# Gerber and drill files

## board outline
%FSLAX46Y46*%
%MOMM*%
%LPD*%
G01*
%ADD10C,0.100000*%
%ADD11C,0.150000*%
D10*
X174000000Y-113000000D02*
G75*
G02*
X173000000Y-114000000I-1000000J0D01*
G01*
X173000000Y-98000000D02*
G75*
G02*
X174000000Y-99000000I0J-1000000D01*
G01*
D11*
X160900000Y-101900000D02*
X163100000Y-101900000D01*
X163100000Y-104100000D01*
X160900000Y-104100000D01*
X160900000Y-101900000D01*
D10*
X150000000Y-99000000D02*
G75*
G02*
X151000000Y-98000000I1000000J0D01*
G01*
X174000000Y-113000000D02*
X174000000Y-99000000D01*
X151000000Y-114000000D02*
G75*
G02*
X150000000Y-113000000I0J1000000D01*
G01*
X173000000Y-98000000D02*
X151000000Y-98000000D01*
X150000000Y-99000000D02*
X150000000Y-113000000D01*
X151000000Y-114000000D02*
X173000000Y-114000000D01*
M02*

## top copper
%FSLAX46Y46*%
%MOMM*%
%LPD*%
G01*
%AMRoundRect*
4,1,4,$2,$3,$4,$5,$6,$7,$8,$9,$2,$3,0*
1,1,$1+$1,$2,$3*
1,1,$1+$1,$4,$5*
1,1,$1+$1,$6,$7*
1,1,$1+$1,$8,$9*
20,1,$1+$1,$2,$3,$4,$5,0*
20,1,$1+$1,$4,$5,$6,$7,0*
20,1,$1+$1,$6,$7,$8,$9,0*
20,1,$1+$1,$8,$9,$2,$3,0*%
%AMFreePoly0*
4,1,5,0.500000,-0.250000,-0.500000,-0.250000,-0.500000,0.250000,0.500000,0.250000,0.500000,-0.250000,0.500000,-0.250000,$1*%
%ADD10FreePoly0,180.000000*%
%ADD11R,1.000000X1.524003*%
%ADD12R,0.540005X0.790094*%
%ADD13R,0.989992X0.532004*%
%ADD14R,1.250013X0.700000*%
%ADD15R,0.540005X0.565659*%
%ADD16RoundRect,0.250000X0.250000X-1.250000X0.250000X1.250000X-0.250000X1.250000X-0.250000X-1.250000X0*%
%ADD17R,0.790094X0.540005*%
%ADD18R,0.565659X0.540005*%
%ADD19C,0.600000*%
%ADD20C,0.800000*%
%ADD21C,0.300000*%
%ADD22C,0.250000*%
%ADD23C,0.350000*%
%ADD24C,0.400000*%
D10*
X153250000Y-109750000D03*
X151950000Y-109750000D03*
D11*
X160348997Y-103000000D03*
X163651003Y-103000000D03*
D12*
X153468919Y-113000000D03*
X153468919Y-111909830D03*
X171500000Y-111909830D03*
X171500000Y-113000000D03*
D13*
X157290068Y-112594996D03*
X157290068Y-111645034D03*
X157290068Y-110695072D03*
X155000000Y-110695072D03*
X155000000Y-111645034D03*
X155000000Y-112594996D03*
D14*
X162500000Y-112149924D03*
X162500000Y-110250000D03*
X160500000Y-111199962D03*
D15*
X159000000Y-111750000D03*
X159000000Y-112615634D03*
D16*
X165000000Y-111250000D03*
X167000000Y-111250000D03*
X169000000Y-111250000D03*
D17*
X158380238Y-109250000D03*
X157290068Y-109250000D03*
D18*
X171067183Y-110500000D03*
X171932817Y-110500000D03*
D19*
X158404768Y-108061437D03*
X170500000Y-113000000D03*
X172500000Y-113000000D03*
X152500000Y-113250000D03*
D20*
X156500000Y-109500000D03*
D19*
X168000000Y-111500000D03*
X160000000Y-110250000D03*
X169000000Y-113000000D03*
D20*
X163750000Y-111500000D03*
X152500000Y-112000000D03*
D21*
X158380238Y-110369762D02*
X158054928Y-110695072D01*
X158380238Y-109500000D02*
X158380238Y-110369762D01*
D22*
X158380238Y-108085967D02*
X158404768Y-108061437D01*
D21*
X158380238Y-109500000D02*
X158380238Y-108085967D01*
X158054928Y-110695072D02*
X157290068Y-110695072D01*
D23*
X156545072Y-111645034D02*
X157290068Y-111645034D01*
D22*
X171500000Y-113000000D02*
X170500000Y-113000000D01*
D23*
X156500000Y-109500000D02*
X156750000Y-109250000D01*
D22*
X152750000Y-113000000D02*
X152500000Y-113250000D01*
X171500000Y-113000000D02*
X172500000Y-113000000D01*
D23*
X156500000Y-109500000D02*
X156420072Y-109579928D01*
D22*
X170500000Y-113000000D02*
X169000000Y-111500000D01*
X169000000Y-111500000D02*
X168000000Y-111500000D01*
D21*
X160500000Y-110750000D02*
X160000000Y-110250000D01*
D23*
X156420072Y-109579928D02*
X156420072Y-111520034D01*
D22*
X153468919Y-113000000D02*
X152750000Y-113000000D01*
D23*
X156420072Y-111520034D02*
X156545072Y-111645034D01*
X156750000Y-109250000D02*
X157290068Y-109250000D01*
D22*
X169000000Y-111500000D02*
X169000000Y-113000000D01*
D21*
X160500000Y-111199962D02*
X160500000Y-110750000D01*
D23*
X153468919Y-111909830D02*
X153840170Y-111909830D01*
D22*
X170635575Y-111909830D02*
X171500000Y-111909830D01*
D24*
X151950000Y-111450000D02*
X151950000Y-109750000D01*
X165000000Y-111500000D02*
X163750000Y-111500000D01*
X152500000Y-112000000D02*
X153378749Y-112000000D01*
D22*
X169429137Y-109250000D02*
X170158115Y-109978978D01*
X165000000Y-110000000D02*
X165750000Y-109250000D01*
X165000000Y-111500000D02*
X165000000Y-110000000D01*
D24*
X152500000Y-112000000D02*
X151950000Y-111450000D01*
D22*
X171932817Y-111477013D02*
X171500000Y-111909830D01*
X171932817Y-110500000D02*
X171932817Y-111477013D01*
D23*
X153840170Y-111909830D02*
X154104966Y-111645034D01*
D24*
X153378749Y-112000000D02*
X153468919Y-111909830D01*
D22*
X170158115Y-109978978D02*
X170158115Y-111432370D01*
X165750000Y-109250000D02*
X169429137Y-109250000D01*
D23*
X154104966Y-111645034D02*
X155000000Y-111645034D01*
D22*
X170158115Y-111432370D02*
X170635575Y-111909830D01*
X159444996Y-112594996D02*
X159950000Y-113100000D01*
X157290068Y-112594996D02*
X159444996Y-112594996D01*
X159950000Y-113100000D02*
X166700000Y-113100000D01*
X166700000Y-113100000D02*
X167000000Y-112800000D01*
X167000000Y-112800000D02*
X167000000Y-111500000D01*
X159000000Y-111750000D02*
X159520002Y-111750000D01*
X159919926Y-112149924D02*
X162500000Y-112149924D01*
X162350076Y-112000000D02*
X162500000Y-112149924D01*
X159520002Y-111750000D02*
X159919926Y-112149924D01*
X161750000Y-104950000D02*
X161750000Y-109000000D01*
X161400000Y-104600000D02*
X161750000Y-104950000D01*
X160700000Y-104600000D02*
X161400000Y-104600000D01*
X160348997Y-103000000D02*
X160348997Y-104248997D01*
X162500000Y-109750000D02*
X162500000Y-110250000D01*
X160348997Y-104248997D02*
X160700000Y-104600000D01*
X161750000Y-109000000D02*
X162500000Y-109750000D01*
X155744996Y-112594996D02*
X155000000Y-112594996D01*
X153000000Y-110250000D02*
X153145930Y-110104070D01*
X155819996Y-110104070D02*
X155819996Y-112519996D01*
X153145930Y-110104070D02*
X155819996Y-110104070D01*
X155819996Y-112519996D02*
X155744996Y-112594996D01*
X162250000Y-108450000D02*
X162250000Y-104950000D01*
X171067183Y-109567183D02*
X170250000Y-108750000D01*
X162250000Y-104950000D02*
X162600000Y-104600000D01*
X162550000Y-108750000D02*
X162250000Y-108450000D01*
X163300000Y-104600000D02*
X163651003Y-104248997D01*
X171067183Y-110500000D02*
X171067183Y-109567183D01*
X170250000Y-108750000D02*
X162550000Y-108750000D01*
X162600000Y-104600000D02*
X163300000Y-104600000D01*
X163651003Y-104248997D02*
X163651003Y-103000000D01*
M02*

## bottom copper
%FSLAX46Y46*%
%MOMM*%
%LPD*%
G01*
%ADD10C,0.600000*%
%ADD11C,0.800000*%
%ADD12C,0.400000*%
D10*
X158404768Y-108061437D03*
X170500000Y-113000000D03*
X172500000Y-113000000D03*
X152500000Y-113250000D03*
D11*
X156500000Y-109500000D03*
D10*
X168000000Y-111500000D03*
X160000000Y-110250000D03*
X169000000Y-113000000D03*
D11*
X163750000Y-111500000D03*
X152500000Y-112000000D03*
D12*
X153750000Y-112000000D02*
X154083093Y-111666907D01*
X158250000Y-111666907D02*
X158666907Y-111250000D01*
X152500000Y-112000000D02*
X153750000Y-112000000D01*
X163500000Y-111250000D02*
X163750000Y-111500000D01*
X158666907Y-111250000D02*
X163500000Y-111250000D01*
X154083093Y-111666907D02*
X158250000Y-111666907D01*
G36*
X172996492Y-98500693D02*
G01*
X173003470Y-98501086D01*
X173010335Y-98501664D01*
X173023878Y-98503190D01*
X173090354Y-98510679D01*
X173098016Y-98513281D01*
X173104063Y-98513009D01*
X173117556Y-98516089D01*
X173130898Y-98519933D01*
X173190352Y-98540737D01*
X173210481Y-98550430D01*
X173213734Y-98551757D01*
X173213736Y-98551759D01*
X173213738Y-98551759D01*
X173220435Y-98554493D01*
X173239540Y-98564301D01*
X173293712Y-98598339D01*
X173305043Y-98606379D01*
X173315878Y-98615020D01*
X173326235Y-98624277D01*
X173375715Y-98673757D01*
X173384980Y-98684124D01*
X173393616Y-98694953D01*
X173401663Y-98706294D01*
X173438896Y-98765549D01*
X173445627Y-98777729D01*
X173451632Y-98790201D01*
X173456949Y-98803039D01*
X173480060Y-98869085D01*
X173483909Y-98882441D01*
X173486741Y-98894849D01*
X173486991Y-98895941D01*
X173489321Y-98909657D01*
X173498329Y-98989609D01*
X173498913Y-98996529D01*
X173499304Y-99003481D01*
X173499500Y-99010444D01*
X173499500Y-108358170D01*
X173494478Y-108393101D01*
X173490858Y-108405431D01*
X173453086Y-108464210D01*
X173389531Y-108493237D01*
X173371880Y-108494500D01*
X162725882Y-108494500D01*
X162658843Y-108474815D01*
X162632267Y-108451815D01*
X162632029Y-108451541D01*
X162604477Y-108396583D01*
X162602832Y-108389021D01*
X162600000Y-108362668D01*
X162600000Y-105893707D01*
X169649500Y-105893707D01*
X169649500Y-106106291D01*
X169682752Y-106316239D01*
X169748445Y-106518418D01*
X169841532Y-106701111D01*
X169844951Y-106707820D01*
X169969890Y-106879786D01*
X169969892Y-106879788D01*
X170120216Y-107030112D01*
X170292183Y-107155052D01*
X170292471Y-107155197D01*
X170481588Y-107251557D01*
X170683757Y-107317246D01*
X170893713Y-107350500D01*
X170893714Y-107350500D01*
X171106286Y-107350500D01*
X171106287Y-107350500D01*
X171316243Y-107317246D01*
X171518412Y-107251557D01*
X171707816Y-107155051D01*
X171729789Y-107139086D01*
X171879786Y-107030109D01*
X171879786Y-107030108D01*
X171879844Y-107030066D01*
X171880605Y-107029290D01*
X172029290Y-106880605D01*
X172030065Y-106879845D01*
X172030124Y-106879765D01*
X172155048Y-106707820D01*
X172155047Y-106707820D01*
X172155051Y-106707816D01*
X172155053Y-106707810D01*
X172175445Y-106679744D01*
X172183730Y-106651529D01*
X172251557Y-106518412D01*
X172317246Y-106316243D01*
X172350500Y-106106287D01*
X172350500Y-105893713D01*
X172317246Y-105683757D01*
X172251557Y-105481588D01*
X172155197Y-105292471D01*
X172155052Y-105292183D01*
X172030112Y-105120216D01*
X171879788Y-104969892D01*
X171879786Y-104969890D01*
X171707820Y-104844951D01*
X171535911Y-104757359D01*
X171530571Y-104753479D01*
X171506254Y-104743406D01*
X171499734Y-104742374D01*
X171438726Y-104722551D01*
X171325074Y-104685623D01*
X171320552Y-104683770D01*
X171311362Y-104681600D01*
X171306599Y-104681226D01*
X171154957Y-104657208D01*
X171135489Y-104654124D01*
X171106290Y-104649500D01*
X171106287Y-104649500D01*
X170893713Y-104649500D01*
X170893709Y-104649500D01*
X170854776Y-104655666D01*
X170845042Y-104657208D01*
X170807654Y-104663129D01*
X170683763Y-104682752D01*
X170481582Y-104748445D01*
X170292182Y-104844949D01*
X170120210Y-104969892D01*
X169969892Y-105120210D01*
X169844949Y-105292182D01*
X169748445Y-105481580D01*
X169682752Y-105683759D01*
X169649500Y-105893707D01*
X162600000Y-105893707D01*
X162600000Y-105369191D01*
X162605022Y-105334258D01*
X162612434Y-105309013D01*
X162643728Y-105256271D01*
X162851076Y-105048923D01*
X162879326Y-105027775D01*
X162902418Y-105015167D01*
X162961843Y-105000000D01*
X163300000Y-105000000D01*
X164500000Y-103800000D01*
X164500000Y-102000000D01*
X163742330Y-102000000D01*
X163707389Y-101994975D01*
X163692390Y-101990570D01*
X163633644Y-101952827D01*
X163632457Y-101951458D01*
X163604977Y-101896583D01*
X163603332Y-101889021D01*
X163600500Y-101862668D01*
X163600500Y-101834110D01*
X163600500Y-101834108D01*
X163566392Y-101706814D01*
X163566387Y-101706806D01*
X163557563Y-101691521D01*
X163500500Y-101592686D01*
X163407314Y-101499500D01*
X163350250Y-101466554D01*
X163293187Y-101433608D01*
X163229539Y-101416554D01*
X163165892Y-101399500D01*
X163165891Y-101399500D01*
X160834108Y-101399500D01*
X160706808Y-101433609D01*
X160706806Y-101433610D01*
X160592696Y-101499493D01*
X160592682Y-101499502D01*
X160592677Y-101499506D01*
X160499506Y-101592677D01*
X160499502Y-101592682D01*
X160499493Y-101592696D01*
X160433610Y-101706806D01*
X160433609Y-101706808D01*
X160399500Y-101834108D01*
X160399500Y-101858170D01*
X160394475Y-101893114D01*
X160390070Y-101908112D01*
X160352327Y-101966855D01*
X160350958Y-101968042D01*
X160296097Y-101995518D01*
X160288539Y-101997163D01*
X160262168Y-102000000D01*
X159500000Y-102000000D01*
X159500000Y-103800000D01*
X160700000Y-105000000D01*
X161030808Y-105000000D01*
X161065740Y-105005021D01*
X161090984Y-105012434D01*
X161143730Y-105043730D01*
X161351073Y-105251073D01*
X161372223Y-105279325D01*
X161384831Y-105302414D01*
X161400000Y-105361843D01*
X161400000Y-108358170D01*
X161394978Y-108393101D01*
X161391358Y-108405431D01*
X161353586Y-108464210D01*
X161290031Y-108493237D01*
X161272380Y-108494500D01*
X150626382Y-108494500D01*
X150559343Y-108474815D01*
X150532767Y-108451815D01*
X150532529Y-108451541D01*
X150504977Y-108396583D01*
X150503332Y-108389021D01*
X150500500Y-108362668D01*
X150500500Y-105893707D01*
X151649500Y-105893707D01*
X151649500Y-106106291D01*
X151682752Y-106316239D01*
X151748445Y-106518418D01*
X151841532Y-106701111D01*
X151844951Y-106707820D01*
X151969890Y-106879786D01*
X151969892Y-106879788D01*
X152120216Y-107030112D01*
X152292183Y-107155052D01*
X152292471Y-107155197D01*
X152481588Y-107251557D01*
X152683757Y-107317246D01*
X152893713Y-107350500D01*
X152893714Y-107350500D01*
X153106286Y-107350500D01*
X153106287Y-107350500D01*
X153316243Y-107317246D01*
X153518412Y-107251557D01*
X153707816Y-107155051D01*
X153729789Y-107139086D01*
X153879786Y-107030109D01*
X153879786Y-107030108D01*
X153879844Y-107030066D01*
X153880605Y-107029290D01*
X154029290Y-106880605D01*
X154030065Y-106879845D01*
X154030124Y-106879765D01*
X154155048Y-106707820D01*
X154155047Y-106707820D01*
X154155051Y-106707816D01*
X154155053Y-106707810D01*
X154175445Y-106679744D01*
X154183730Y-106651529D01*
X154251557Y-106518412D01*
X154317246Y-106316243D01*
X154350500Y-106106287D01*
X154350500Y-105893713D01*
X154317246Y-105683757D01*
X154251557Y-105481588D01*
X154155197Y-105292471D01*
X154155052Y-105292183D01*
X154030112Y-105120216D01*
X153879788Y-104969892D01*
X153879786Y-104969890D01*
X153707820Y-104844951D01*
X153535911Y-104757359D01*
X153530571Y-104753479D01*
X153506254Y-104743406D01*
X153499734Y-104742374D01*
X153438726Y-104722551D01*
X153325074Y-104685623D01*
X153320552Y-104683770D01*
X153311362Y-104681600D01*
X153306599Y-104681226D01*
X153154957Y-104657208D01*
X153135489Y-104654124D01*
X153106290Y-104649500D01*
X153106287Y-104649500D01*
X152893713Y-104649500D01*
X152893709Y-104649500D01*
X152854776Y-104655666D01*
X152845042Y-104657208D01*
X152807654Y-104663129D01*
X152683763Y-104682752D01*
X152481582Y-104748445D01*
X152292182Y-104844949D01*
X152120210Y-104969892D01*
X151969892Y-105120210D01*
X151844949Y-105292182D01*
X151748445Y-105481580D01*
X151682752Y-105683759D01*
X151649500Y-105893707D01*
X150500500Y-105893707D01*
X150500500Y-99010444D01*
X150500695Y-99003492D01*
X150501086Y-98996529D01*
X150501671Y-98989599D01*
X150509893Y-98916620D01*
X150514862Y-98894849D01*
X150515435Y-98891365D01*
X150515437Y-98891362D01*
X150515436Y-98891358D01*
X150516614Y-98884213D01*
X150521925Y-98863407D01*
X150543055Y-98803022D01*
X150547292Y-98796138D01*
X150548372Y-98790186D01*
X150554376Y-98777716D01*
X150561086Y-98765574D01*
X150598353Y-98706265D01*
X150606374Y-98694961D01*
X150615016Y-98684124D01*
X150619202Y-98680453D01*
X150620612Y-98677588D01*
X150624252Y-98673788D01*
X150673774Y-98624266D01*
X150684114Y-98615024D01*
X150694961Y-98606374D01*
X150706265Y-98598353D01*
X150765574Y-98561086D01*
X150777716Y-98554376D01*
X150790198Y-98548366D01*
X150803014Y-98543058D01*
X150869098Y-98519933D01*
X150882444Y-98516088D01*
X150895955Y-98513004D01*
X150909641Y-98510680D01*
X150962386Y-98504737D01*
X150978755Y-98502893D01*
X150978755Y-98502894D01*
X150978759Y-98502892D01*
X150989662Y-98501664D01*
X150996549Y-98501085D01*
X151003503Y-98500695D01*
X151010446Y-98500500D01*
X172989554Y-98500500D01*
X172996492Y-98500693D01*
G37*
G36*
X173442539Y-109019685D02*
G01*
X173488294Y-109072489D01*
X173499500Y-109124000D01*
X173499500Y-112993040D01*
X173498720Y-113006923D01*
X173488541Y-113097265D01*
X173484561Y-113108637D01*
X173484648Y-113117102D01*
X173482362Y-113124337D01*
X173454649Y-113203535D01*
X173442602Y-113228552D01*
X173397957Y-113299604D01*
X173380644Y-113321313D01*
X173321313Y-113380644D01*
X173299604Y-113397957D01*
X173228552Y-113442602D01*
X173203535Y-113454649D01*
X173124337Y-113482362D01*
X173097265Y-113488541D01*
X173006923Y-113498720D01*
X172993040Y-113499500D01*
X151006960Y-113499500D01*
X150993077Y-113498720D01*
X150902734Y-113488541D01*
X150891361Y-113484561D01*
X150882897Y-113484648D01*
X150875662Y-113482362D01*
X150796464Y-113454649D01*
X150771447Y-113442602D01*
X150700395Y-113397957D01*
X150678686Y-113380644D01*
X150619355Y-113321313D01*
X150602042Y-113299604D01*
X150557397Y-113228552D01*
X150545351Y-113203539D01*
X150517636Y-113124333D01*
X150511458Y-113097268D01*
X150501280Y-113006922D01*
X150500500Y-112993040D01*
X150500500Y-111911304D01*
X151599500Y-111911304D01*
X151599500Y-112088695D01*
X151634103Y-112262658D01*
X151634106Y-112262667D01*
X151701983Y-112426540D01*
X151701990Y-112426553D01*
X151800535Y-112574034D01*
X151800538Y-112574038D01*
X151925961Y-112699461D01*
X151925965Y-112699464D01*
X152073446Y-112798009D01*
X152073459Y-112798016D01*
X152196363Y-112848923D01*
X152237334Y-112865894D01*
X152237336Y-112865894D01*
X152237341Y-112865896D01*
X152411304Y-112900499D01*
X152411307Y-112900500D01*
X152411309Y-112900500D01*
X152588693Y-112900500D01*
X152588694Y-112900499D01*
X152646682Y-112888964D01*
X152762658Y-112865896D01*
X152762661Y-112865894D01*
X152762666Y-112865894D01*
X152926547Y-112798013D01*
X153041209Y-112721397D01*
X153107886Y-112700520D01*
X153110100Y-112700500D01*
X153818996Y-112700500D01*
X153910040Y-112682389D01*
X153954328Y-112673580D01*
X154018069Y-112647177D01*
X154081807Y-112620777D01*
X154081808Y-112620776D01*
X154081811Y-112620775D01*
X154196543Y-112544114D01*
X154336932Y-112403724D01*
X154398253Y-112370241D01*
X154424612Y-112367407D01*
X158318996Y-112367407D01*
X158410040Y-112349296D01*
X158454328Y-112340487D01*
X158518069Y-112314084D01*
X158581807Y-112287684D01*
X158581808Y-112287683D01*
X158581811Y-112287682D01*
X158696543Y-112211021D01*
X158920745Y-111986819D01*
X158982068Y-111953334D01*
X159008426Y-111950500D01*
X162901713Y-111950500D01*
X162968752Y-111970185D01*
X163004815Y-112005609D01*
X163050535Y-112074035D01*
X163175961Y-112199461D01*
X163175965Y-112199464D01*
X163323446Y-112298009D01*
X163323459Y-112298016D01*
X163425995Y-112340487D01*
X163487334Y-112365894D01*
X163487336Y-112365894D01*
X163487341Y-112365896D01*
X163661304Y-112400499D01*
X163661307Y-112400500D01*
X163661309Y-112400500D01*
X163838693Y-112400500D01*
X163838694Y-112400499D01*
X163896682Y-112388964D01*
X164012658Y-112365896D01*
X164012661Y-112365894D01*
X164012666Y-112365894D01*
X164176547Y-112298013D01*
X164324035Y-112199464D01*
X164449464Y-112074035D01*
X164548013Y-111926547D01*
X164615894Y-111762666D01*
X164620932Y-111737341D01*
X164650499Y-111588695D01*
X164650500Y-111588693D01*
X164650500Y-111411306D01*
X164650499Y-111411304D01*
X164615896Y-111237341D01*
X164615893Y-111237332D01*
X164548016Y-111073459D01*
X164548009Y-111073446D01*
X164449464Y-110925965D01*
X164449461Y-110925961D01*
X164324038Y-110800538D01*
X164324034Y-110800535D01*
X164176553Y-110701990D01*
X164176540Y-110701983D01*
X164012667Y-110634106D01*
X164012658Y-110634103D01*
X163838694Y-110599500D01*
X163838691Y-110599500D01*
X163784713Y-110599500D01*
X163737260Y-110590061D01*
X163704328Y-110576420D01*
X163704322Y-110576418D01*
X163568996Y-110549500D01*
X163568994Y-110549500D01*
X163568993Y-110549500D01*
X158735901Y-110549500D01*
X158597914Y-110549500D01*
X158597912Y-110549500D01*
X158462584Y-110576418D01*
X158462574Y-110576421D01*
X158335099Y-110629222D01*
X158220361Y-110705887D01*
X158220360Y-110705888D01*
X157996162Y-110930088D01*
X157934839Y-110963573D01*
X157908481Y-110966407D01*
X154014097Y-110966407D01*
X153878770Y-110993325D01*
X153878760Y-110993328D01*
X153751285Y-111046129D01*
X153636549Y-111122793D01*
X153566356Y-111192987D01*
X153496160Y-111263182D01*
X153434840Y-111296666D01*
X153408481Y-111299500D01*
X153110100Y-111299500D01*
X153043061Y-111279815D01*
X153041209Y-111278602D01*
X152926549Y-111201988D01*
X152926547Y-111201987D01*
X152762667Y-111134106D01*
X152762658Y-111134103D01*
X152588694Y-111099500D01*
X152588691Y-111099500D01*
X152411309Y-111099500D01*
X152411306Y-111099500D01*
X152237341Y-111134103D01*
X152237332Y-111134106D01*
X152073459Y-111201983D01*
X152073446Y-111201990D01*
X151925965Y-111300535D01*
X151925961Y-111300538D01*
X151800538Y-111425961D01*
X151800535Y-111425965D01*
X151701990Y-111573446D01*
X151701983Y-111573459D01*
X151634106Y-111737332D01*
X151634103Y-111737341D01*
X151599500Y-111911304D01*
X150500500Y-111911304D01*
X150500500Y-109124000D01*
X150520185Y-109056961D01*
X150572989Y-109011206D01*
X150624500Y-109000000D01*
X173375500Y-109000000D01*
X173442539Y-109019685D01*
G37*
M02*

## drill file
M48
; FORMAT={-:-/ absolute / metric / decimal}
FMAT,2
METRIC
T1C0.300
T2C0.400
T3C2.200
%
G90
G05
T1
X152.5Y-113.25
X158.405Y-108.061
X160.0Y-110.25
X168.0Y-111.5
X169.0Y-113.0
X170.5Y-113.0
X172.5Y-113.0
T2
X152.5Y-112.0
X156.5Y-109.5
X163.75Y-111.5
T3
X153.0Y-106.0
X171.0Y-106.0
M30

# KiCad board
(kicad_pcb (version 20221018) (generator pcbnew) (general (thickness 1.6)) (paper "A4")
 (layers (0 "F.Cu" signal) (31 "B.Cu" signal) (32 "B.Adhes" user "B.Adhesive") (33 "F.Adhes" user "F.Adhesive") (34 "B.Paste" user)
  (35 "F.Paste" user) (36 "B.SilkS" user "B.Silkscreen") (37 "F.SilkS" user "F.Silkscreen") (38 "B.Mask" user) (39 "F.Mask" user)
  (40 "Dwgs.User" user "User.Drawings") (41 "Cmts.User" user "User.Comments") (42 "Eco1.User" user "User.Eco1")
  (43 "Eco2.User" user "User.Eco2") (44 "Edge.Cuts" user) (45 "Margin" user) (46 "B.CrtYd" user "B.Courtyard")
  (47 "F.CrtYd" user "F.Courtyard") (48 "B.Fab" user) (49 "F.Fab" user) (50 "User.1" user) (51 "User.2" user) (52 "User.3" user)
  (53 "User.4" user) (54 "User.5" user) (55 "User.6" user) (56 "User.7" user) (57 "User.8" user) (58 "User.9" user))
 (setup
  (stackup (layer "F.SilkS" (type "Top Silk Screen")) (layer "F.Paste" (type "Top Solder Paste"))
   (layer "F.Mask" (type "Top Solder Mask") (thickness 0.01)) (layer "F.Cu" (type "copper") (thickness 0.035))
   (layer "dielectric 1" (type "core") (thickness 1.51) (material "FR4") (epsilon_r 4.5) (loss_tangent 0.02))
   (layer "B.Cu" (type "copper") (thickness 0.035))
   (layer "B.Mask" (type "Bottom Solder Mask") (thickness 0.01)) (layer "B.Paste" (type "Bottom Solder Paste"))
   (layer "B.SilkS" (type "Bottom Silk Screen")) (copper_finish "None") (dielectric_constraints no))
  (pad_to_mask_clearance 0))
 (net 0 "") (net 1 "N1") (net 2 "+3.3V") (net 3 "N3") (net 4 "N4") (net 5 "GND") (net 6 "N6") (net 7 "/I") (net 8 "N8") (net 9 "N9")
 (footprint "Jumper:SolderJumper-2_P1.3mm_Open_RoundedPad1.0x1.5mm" (layer "F.Cu") (at 152.6 109.75 180)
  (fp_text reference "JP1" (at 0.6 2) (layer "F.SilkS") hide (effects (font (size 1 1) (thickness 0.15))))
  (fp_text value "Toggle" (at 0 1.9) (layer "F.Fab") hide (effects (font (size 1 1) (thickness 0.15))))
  (pad "1" smd custom (at -0.65 0 180) (size 1 0.5) (layers "F.Cu" "F.Mask") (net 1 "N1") (zone_connect 2) (thermal_bridge_angle 45)
   (options (clearance outline) (anchor rect)) (primitives))
  (pad "2" smd custom (at 0.65 0 180) (size 1 0.5) (layers "F.Cu" "F.Mask") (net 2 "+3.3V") (zone_connect 2) (thermal_bridge_angle 45)
   (options (clearance outline) (anchor rect)) (primitives)))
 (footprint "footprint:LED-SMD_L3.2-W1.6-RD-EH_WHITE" (layer "F.Cu") (at 162 103)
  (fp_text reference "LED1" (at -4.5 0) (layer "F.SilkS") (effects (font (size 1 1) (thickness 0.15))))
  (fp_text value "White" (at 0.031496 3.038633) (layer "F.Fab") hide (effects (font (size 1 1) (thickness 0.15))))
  (pad "1" smd rect (at -1.651003 0) (size 1 1.524003) (layers "F.Cu" "F.Paste" "F.Mask") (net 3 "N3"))
  (pad "2" smd rect (at 1.651003 0) (size 1 1.524003) (layers "F.Cu" "F.Paste" "F.Mask") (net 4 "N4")))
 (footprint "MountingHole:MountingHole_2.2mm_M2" (layer "F.Cu") (at 153 106)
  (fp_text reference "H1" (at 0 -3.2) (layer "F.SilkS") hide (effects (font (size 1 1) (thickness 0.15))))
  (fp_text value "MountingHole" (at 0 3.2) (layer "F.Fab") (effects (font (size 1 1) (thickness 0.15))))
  (pad "" np_thru_hole circle (at 0 0) (size 2.2 2.2) (drill 2.2) (layers "*.Cu" "*.Mask")))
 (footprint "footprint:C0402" (layer "F.Cu") (at 153.468919 112.454915 90)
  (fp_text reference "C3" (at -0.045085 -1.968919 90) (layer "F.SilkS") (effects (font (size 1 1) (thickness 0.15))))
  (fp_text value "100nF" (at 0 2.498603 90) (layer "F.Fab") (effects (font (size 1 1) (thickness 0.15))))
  (pad "1" smd rect (at -0.545085 0 90) (size 0.790094 0.540005) (layers "F.Cu" "F.Paste" "F.Mask") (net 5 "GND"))
  (pad "2" smd rect (at 0.545085 0 90) (size 0.790094 0.540005) (layers "F.Cu" "F.Paste" "F.Mask") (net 2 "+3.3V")))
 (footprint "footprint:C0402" (layer "F.Cu") (at 171.5 112.454915 -90)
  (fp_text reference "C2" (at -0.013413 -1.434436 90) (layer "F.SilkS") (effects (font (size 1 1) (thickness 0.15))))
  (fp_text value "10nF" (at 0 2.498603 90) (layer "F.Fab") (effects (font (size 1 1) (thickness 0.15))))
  (pad "1" smd rect (at -0.545085 0 270) (size 0.790094 0.540005) (layers "F.Cu" "F.Paste" "F.Mask") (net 2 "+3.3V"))
  (pad "2" smd rect (at 0.545085 0 270) (size 0.790094 0.540005) (layers "F.Cu" "F.Paste" "F.Mask") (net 5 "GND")))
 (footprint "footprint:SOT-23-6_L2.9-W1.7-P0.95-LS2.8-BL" (layer "F.Cu") (at 156.145034 111.645034 90)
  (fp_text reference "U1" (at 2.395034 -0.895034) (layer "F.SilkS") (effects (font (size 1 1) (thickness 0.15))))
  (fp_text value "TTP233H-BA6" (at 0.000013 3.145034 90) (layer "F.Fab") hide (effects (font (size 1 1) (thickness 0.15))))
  (pad "1" smd rect (at -0.949962 1.145034 90) (size 0.532004 0.989992) (layers "F.Cu" "F.Paste" "F.Mask") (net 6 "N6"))
  (pad "2" smd rect (at 0 1.145034 90) (size 0.532004 0.989992) (layers "F.Cu" "F.Paste" "F.Mask") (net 5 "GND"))
  (pad "3" smd rect (at 0.949962 1.145034 90) (size 0.532004 0.989992) (layers "F.Cu" "F.Paste" "F.Mask") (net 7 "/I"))
  (pad "4" smd rect (at 0.949962 -1.145034 90) (size 0.532004 0.989992) (layers "F.Cu" "F.Paste" "F.Mask") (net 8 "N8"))
  (pad "5" smd rect (at 0 -1.145034 90) (size 0.532004 0.989992) (layers "F.Cu" "F.Paste" "F.Mask") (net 2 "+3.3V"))
  (pad "6" smd rect (at -0.949962 -1.145034 90) (size 0.532004 0.989992) (layers "F.Cu" "F.Paste" "F.Mask") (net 1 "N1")))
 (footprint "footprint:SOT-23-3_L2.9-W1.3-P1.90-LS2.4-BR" (layer "F.Cu") (at 161.5 111.199962)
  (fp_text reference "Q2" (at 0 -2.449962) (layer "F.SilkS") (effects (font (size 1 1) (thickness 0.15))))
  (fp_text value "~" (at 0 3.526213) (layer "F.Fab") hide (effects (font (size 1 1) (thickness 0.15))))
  (pad "1" smd rect (at 1 0.949962) (size 1.250013 0.7) (layers "F.Cu" "F.Paste" "F.Mask") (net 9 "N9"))
  (pad "2" smd rect (at 1 -0.949962) (size 1.250013 0.7) (layers "F.Cu" "F.Paste" "F.Mask") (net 3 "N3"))
  (pad "3" smd rect (at -1 0) (size 1.250013 0.7) (layers "F.Cu" "F.Paste" "F.Mask") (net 5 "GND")))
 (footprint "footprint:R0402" (layer "F.Cu") (at 159 112.182817 -90)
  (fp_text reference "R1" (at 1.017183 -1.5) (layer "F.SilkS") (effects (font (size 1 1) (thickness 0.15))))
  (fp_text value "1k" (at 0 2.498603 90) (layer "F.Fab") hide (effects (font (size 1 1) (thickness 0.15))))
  (pad "1" smd rect (at -0.432817 0 270) (size 0.565659 0.540005) (layers "F.Cu" "F.Paste" "F.Mask") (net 9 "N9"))
  (pad "2" smd rect (at 0.432817 0 270) (size 0.565659 0.540005) (layers "F.Cu" "F.Paste" "F.Mask") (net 6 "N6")))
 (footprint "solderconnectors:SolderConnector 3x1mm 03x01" (layer "F.Cu") (at 167 111.25 90)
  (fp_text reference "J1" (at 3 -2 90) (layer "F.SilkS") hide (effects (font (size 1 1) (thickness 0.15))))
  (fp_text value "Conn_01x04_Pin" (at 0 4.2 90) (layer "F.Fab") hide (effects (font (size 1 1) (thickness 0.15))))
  (pad "1" smd roundrect (at 0 -2 90) (size 3 1) (layers "F.Cu" "F.Mask") (roundrect_rratio 0.25) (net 2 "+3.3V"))
  (pad "2" smd roundrect (at 0 0 90) (size 3 1) (layers "F.Cu" "F.Mask") (roundrect_rratio 0.25) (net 6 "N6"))
  (pad "3" smd roundrect (at 0 2 90) (size 3 1) (layers "F.Cu" "F.Mask") (roundrect_rratio 0.25) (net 5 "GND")))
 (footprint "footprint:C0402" (layer "F.Cu") (at 157.835153 109.25 180)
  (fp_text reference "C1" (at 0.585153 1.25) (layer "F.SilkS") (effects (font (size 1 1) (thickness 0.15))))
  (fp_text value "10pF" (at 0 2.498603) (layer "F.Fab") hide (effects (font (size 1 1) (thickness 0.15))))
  (pad "1" smd rect (at -0.545085 0 180) (size 0.790094 0.540005) (layers "F.Cu" "F.Paste" "F.Mask") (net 7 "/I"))
  (pad "2" smd rect (at 0.545085 0 180) (size 0.790094 0.540005) (layers "F.Cu" "F.Paste" "F.Mask") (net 5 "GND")))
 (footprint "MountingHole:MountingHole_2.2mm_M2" (layer "F.Cu") (at 171 106)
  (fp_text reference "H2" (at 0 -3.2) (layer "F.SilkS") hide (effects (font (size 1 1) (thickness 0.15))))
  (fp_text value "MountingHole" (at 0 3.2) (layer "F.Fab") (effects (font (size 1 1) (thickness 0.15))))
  (pad "" np_thru_hole circle (at 0 0) (size 2.2 2.2) (drill 2.2) (layers "*.Cu" "*.Mask")))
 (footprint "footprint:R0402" (layer "F.Cu") (at 171.5 110.5)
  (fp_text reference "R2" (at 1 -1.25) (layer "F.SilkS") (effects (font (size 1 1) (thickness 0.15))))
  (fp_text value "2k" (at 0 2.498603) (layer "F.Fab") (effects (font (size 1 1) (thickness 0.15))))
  (pad "1" smd rect (at -0.432817 0) (size 0.565659 0.540005) (layers "F.Cu" "F.Paste" "F.Mask") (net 4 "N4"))
  (pad "2" smd rect (at 0.432817 0) (size 0.565659 0.540005) (layers "F.Cu" "F.Paste" "F.Mask") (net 2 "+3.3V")))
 (gr_arc (start 174 113) (mid 173.707107 113.707107) (end 173 114) (stroke (width 0.1) (type default)) (layer "Edge.Cuts"))
 (gr_arc (start 173 98) (mid 173.707107 98.292893) (end 174 99) (stroke (width 0.1) (type default)) (layer "Edge.Cuts"))
 (gr_rect (start 160.9 101.9) (end 163.1 104.1) (stroke (width 0.15) (type solid)) (fill none) (layer "Edge.Cuts"))
 (gr_arc (start 150 99) (mid 150.292893 98.292893) (end 151 98) (stroke (width 0.1) (type default)) (layer "Edge.Cuts"))
 (gr_line (start 174 113) (end 174 99) (stroke (width 0.1) (type default)) (layer "Edge.Cuts"))
 (gr_arc (start 151 114) (mid 150.292893 113.707107) (end 150 113) (stroke (width 0.1) (type default)) (layer "Edge.Cuts"))
 (gr_line (start 173 98) (end 151 98) (stroke (width 0.1) (type default)) (layer "Edge.Cuts"))
 (gr_line (start 150 99) (end 150 113) (stroke (width 0.1) (type default)) (layer "Edge.Cuts"))
 (gr_line (start 151 114) (end 173 114) (stroke (width 0.1) (type default)) (layer "Edge.Cuts"))
 (segment (start 158.380238 110.369762) (end 158.054928 110.695072) (width 0.3) (layer "F.Cu") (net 7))
 (segment (start 158.380238 109.5) (end 158.380238 110.369762) (width 0.3) (layer "F.Cu") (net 7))
 (segment (start 158.380238 108.085967) (end 158.404768 108.061437) (width 0.25) (layer "F.Cu") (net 7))
 (segment (start 158.380238 109.5) (end 158.380238 108.085967) (width 0.3) (layer "F.Cu") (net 7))
 (segment (start 158.054928 110.695072) (end 157.290068 110.695072) (width 0.3) (layer "F.Cu") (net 7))
 (via (at 158.404768 108.061437) (size 0.6) (drill 0.3) (layers "F.Cu" "B.Cu") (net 7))
 (segment (start 156.545072 111.645034) (end 157.290068 111.645034) (width 0.35) (layer "F.Cu") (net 5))
 (segment (start 171.5 113) (end 170.5 113) (width 0.25) (layer "F.Cu") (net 5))
 (segment (start 156.5 109.5) (end 156.75 109.25) (width 0.35) (layer "F.Cu") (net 5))
 (segment (start 152.75 113) (end 152.5 113.25) (width 0.25) (layer "F.Cu") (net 5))
 (segment (start 171.5 113) (end 172.5 113) (width 0.25) (layer "F.Cu") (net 5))
 (segment (start 156.5 109.5) (end 156.420072 109.579928) (width 0.35) (layer "F.Cu") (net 5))
 (segment (start 170.5 113) (end 169 111.5) (width 0.25) (layer "F.Cu") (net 5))
 (segment (start 169 111.5) (end 168 111.5) (width 0.25) (layer "F.Cu") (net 5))
 (segment (start 160.5 110.75) (end 160 110.25) (width 0.3) (layer "F.Cu") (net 5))
 (segment (start 156.420072 109.579928) (end 156.420072 111.520034) (width 0.35) (layer "F.Cu") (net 5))
 (segment (start 153.468919 113) (end 152.75 113) (width 0.25) (layer "F.Cu") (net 5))
 (segment (start 156.420072 111.520034) (end 156.545072 111.645034) (width 0.35) (layer "F.Cu") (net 5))
 (segment (start 156.75 109.25) (end 157.290068 109.25) (width 0.35) (layer "F.Cu") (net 5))
 (segment (start 169 111.5) (end 169 113) (width 0.25) (layer "F.Cu") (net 5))
 (segment (start 160.5 111.199962) (end 160.5 110.75) (width 0.3) (layer "F.Cu") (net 5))
 (via (at 170.5 113) (size 0.6) (drill 0.3) (layers "F.Cu" "B.Cu") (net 5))
 (via (at 172.5 113) (size 0.6) (drill 0.3) (layers "F.Cu" "B.Cu") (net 5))
 (via (at 152.5 113.25) (size 0.6) (drill 0.3) (layers "F.Cu" "B.Cu") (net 5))
 (via (at 156.5 109.5) (size 0.8) (drill 0.4) (layers "F.Cu" "B.Cu") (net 5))
 (via (at 168 111.5) (size 0.6) (drill 0.3) (layers "F.Cu" "B.Cu") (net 5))
 (via (at 160 110.25) (size 0.6) (drill 0.3) (layers "F.Cu" "B.Cu") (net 5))
 (via (at 169 113) (size 0.6) (drill 0.3) (layers "F.Cu" "B.Cu") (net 5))
 (segment (start 153.468919 111.90983) (end 153.84017 111.90983) (width 0.35) (layer "F.Cu") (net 2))
 (segment (start 170.635575 111.90983) (end 171.5 111.90983) (width 0.25) (layer "F.Cu") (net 2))
 (segment (start 151.95 111.45) (end 151.95 109.75) (width 0.4) (layer "F.Cu") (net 2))
 (segment (start 165 111.5) (end 163.75 111.5) (width 0.4) (layer "F.Cu") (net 2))
 (segment (start 152.5 112) (end 153.378749 112) (width 0.4) (layer "F.Cu") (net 2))
 (segment (start 169.429137 109.25) (end 170.158115 109.978978) (width 0.25) (layer "F.Cu") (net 2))
 (segment (start 165 110) (end 165.75 109.25) (width 0.25) (layer "F.Cu") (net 2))
 (segment (start 165 111.5) (end 165 110) (width 0.25) (layer "F.Cu") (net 2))
 (segment (start 152.5 112) (end 151.95 111.45) (width 0.4) (layer "F.Cu") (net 2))
 (segment (start 171.932817 111.477013) (end 171.5 111.90983) (width 0.25) (layer "F.Cu") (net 2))
 (segment (start 171.932817 110.5) (end 171.932817 111.477013) (width 0.25) (layer "F.Cu") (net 2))
 (segment (start 153.84017 111.90983) (end 154.104966 111.645034) (width 0.35) (layer "F.Cu") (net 2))
 (segment (start 153.378749 112) (end 153.468919 111.90983) (width 0.4) (layer "F.Cu") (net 2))
 (segment (start 170.158115 109.978978) (end 170.158115 111.43237) (width 0.25) (layer "F.Cu") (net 2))
 (segment (start 165.75 109.25) (end 169.429137 109.25) (width 0.25) (layer "F.Cu") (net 2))
 (segment (start 154.104966 111.645034) (end 155 111.645034) (width 0.35) (layer "F.Cu") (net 2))
 (segment (start 170.158115 111.43237) (end 170.635575 111.90983) (width 0.25) (layer "F.Cu") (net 2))
 (via (at 163.75 111.5) (size 0.8) (drill 0.4) (layers "F.Cu" "B.Cu") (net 2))
 (via (at 152.5 112) (size 0.8) (drill 0.4) (layers "F.Cu" "B.Cu") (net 2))
 (segment (start 153.75 112) (end 154.083093 111.666907) (width 0.4) (layer "B.Cu") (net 2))
 (segment (start 158.25 111.666907) (end 158.666907 111.25) (width 0.4) (layer "B.Cu") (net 2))
 (segment (start 152.5 112) (end 153.75 112) (width 0.4) (layer "B.Cu") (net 2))
 (segment (start 163.5 111.25) (end 163.75 111.5) (width 0.4) (layer "B.Cu") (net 2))
 (segment (start 158.666907 111.25) (end 163.5 111.25) (width 0.4) (layer "B.Cu") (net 2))
 (segment (start 154.083093 111.666907) (end 158.25 111.666907) (width 0.4) (layer "B.Cu") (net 2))
 (segment (start 159.444996 112.594996) (end 159.95 113.1) (width 0.25) (layer "F.Cu") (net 6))
 (segment (start 157.290068 112.594996) (end 159.444996 112.594996) (width 0.25) (layer "F.Cu") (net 6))
 (segment (start 159.95 113.1) (end 166.7 113.1) (width 0.25) (layer "F.Cu") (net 6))
 (segment (start 166.7 113.1) (end 167 112.8) (width 0.25) (layer "F.Cu") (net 6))
 (segment (start 167 112.8) (end 167 111.5) (width 0.25) (layer "F.Cu") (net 6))
 (segment (start 159 111.75) (end 159.520002 111.75) (width 0.25) (layer "F.Cu") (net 9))
 (segment (start 159.919926 112.149924) (end 162.5 112.149924) (width 0.25) (layer "F.Cu") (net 9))
 (segment (start 162.350076 112) (end 162.5 112.149924) (width 0.25) (layer "F.Cu") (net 9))
 (segment (start 159.520002 111.75) (end 159.919926 112.149924) (width 0.25) (layer "F.Cu") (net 9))
 (segment (start 161.75 104.95) (end 161.75 109) (width 0.25) (layer "F.Cu") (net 3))
 (segment (start 161.4 104.6) (end 161.75 104.95) (width 0.25) (layer "F.Cu") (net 3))
 (segment (start 160.7 104.6) (end 161.4 104.6) (width 0.25) (layer "F.Cu") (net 3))
 (segment (start 160.348997 103) (end 160.348997 104.248997) (width 0.25) (layer "F.Cu") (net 3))
 (segment (start 162.5 109.75) (end 162.5 110.25) (width 0.25) (layer "F.Cu") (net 3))
 (segment (start 160.348997 104.248997) (end 160.7 104.6) (width 0.25) (layer "F.Cu") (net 3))
 (segment (start 161.75 109) (end 162.5 109.75) (width 0.25) (layer "F.Cu") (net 3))
 (segment (start 155.744996 112.594996) (end 155 112.594996) (width 0.25) (layer "F.Cu") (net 1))
 (segment (start 153 110.25) (end 153.14593 110.10407) (width 0.25) (layer "F.Cu") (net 1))
 (segment (start 155.819996 110.10407) (end 155.819996 112.519996) (width 0.25) (layer "F.Cu") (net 1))
 (segment (start 153.14593 110.10407) (end 155.819996 110.10407) (width 0.25) (layer "F.Cu") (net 1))
 (segment (start 155.819996 112.519996) (end 155.744996 112.594996) (width 0.25) (layer "F.Cu") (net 1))
 (segment (start 162.25 108.45) (end 162.25 104.95) (width 0.25) (layer "F.Cu") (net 4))
 (segment (start 171.067183 109.567183) (end 170.25 108.75) (width 0.25) (layer "F.Cu") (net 4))
 (segment (start 162.25 104.95) (end 162.6 104.6) (width 0.25) (layer "F.Cu") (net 4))
 (segment (start 162.55 108.75) (end 162.25 108.45) (width 0.25) (layer "F.Cu") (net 4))
 (segment (start 163.3 104.6) (end 163.651003 104.248997) (width 0.25) (layer "F.Cu") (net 4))
 (segment (start 171.067183 110.5) (end 171.067183 109.567183) (width 0.25) (layer "F.Cu") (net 4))
 (segment (start 170.25 108.75) (end 162.55 108.75) (width 0.25) (layer "F.Cu") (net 4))
 (segment (start 162.6 104.6) (end 163.3 104.6) (width 0.25) (layer "F.Cu") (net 4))
 (segment (start 163.651003 104.248997) (end 163.651003 103) (width 0.25) (layer "F.Cu") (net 4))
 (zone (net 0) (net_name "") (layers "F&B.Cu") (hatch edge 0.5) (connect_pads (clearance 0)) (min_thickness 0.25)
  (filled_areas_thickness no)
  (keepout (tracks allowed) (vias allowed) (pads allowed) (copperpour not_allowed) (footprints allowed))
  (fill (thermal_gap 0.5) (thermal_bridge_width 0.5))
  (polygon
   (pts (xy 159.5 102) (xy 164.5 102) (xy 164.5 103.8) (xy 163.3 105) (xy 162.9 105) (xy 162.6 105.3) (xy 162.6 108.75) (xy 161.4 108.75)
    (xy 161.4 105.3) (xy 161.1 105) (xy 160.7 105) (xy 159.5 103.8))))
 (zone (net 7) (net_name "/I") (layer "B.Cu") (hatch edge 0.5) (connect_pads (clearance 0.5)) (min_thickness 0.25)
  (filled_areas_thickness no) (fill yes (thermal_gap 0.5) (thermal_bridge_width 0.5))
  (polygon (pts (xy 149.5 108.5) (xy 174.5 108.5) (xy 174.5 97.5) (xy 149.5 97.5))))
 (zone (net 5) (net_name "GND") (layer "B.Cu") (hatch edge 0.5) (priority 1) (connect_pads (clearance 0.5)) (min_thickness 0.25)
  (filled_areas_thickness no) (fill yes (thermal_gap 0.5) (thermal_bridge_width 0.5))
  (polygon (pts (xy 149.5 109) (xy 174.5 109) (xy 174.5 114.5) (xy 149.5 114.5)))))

